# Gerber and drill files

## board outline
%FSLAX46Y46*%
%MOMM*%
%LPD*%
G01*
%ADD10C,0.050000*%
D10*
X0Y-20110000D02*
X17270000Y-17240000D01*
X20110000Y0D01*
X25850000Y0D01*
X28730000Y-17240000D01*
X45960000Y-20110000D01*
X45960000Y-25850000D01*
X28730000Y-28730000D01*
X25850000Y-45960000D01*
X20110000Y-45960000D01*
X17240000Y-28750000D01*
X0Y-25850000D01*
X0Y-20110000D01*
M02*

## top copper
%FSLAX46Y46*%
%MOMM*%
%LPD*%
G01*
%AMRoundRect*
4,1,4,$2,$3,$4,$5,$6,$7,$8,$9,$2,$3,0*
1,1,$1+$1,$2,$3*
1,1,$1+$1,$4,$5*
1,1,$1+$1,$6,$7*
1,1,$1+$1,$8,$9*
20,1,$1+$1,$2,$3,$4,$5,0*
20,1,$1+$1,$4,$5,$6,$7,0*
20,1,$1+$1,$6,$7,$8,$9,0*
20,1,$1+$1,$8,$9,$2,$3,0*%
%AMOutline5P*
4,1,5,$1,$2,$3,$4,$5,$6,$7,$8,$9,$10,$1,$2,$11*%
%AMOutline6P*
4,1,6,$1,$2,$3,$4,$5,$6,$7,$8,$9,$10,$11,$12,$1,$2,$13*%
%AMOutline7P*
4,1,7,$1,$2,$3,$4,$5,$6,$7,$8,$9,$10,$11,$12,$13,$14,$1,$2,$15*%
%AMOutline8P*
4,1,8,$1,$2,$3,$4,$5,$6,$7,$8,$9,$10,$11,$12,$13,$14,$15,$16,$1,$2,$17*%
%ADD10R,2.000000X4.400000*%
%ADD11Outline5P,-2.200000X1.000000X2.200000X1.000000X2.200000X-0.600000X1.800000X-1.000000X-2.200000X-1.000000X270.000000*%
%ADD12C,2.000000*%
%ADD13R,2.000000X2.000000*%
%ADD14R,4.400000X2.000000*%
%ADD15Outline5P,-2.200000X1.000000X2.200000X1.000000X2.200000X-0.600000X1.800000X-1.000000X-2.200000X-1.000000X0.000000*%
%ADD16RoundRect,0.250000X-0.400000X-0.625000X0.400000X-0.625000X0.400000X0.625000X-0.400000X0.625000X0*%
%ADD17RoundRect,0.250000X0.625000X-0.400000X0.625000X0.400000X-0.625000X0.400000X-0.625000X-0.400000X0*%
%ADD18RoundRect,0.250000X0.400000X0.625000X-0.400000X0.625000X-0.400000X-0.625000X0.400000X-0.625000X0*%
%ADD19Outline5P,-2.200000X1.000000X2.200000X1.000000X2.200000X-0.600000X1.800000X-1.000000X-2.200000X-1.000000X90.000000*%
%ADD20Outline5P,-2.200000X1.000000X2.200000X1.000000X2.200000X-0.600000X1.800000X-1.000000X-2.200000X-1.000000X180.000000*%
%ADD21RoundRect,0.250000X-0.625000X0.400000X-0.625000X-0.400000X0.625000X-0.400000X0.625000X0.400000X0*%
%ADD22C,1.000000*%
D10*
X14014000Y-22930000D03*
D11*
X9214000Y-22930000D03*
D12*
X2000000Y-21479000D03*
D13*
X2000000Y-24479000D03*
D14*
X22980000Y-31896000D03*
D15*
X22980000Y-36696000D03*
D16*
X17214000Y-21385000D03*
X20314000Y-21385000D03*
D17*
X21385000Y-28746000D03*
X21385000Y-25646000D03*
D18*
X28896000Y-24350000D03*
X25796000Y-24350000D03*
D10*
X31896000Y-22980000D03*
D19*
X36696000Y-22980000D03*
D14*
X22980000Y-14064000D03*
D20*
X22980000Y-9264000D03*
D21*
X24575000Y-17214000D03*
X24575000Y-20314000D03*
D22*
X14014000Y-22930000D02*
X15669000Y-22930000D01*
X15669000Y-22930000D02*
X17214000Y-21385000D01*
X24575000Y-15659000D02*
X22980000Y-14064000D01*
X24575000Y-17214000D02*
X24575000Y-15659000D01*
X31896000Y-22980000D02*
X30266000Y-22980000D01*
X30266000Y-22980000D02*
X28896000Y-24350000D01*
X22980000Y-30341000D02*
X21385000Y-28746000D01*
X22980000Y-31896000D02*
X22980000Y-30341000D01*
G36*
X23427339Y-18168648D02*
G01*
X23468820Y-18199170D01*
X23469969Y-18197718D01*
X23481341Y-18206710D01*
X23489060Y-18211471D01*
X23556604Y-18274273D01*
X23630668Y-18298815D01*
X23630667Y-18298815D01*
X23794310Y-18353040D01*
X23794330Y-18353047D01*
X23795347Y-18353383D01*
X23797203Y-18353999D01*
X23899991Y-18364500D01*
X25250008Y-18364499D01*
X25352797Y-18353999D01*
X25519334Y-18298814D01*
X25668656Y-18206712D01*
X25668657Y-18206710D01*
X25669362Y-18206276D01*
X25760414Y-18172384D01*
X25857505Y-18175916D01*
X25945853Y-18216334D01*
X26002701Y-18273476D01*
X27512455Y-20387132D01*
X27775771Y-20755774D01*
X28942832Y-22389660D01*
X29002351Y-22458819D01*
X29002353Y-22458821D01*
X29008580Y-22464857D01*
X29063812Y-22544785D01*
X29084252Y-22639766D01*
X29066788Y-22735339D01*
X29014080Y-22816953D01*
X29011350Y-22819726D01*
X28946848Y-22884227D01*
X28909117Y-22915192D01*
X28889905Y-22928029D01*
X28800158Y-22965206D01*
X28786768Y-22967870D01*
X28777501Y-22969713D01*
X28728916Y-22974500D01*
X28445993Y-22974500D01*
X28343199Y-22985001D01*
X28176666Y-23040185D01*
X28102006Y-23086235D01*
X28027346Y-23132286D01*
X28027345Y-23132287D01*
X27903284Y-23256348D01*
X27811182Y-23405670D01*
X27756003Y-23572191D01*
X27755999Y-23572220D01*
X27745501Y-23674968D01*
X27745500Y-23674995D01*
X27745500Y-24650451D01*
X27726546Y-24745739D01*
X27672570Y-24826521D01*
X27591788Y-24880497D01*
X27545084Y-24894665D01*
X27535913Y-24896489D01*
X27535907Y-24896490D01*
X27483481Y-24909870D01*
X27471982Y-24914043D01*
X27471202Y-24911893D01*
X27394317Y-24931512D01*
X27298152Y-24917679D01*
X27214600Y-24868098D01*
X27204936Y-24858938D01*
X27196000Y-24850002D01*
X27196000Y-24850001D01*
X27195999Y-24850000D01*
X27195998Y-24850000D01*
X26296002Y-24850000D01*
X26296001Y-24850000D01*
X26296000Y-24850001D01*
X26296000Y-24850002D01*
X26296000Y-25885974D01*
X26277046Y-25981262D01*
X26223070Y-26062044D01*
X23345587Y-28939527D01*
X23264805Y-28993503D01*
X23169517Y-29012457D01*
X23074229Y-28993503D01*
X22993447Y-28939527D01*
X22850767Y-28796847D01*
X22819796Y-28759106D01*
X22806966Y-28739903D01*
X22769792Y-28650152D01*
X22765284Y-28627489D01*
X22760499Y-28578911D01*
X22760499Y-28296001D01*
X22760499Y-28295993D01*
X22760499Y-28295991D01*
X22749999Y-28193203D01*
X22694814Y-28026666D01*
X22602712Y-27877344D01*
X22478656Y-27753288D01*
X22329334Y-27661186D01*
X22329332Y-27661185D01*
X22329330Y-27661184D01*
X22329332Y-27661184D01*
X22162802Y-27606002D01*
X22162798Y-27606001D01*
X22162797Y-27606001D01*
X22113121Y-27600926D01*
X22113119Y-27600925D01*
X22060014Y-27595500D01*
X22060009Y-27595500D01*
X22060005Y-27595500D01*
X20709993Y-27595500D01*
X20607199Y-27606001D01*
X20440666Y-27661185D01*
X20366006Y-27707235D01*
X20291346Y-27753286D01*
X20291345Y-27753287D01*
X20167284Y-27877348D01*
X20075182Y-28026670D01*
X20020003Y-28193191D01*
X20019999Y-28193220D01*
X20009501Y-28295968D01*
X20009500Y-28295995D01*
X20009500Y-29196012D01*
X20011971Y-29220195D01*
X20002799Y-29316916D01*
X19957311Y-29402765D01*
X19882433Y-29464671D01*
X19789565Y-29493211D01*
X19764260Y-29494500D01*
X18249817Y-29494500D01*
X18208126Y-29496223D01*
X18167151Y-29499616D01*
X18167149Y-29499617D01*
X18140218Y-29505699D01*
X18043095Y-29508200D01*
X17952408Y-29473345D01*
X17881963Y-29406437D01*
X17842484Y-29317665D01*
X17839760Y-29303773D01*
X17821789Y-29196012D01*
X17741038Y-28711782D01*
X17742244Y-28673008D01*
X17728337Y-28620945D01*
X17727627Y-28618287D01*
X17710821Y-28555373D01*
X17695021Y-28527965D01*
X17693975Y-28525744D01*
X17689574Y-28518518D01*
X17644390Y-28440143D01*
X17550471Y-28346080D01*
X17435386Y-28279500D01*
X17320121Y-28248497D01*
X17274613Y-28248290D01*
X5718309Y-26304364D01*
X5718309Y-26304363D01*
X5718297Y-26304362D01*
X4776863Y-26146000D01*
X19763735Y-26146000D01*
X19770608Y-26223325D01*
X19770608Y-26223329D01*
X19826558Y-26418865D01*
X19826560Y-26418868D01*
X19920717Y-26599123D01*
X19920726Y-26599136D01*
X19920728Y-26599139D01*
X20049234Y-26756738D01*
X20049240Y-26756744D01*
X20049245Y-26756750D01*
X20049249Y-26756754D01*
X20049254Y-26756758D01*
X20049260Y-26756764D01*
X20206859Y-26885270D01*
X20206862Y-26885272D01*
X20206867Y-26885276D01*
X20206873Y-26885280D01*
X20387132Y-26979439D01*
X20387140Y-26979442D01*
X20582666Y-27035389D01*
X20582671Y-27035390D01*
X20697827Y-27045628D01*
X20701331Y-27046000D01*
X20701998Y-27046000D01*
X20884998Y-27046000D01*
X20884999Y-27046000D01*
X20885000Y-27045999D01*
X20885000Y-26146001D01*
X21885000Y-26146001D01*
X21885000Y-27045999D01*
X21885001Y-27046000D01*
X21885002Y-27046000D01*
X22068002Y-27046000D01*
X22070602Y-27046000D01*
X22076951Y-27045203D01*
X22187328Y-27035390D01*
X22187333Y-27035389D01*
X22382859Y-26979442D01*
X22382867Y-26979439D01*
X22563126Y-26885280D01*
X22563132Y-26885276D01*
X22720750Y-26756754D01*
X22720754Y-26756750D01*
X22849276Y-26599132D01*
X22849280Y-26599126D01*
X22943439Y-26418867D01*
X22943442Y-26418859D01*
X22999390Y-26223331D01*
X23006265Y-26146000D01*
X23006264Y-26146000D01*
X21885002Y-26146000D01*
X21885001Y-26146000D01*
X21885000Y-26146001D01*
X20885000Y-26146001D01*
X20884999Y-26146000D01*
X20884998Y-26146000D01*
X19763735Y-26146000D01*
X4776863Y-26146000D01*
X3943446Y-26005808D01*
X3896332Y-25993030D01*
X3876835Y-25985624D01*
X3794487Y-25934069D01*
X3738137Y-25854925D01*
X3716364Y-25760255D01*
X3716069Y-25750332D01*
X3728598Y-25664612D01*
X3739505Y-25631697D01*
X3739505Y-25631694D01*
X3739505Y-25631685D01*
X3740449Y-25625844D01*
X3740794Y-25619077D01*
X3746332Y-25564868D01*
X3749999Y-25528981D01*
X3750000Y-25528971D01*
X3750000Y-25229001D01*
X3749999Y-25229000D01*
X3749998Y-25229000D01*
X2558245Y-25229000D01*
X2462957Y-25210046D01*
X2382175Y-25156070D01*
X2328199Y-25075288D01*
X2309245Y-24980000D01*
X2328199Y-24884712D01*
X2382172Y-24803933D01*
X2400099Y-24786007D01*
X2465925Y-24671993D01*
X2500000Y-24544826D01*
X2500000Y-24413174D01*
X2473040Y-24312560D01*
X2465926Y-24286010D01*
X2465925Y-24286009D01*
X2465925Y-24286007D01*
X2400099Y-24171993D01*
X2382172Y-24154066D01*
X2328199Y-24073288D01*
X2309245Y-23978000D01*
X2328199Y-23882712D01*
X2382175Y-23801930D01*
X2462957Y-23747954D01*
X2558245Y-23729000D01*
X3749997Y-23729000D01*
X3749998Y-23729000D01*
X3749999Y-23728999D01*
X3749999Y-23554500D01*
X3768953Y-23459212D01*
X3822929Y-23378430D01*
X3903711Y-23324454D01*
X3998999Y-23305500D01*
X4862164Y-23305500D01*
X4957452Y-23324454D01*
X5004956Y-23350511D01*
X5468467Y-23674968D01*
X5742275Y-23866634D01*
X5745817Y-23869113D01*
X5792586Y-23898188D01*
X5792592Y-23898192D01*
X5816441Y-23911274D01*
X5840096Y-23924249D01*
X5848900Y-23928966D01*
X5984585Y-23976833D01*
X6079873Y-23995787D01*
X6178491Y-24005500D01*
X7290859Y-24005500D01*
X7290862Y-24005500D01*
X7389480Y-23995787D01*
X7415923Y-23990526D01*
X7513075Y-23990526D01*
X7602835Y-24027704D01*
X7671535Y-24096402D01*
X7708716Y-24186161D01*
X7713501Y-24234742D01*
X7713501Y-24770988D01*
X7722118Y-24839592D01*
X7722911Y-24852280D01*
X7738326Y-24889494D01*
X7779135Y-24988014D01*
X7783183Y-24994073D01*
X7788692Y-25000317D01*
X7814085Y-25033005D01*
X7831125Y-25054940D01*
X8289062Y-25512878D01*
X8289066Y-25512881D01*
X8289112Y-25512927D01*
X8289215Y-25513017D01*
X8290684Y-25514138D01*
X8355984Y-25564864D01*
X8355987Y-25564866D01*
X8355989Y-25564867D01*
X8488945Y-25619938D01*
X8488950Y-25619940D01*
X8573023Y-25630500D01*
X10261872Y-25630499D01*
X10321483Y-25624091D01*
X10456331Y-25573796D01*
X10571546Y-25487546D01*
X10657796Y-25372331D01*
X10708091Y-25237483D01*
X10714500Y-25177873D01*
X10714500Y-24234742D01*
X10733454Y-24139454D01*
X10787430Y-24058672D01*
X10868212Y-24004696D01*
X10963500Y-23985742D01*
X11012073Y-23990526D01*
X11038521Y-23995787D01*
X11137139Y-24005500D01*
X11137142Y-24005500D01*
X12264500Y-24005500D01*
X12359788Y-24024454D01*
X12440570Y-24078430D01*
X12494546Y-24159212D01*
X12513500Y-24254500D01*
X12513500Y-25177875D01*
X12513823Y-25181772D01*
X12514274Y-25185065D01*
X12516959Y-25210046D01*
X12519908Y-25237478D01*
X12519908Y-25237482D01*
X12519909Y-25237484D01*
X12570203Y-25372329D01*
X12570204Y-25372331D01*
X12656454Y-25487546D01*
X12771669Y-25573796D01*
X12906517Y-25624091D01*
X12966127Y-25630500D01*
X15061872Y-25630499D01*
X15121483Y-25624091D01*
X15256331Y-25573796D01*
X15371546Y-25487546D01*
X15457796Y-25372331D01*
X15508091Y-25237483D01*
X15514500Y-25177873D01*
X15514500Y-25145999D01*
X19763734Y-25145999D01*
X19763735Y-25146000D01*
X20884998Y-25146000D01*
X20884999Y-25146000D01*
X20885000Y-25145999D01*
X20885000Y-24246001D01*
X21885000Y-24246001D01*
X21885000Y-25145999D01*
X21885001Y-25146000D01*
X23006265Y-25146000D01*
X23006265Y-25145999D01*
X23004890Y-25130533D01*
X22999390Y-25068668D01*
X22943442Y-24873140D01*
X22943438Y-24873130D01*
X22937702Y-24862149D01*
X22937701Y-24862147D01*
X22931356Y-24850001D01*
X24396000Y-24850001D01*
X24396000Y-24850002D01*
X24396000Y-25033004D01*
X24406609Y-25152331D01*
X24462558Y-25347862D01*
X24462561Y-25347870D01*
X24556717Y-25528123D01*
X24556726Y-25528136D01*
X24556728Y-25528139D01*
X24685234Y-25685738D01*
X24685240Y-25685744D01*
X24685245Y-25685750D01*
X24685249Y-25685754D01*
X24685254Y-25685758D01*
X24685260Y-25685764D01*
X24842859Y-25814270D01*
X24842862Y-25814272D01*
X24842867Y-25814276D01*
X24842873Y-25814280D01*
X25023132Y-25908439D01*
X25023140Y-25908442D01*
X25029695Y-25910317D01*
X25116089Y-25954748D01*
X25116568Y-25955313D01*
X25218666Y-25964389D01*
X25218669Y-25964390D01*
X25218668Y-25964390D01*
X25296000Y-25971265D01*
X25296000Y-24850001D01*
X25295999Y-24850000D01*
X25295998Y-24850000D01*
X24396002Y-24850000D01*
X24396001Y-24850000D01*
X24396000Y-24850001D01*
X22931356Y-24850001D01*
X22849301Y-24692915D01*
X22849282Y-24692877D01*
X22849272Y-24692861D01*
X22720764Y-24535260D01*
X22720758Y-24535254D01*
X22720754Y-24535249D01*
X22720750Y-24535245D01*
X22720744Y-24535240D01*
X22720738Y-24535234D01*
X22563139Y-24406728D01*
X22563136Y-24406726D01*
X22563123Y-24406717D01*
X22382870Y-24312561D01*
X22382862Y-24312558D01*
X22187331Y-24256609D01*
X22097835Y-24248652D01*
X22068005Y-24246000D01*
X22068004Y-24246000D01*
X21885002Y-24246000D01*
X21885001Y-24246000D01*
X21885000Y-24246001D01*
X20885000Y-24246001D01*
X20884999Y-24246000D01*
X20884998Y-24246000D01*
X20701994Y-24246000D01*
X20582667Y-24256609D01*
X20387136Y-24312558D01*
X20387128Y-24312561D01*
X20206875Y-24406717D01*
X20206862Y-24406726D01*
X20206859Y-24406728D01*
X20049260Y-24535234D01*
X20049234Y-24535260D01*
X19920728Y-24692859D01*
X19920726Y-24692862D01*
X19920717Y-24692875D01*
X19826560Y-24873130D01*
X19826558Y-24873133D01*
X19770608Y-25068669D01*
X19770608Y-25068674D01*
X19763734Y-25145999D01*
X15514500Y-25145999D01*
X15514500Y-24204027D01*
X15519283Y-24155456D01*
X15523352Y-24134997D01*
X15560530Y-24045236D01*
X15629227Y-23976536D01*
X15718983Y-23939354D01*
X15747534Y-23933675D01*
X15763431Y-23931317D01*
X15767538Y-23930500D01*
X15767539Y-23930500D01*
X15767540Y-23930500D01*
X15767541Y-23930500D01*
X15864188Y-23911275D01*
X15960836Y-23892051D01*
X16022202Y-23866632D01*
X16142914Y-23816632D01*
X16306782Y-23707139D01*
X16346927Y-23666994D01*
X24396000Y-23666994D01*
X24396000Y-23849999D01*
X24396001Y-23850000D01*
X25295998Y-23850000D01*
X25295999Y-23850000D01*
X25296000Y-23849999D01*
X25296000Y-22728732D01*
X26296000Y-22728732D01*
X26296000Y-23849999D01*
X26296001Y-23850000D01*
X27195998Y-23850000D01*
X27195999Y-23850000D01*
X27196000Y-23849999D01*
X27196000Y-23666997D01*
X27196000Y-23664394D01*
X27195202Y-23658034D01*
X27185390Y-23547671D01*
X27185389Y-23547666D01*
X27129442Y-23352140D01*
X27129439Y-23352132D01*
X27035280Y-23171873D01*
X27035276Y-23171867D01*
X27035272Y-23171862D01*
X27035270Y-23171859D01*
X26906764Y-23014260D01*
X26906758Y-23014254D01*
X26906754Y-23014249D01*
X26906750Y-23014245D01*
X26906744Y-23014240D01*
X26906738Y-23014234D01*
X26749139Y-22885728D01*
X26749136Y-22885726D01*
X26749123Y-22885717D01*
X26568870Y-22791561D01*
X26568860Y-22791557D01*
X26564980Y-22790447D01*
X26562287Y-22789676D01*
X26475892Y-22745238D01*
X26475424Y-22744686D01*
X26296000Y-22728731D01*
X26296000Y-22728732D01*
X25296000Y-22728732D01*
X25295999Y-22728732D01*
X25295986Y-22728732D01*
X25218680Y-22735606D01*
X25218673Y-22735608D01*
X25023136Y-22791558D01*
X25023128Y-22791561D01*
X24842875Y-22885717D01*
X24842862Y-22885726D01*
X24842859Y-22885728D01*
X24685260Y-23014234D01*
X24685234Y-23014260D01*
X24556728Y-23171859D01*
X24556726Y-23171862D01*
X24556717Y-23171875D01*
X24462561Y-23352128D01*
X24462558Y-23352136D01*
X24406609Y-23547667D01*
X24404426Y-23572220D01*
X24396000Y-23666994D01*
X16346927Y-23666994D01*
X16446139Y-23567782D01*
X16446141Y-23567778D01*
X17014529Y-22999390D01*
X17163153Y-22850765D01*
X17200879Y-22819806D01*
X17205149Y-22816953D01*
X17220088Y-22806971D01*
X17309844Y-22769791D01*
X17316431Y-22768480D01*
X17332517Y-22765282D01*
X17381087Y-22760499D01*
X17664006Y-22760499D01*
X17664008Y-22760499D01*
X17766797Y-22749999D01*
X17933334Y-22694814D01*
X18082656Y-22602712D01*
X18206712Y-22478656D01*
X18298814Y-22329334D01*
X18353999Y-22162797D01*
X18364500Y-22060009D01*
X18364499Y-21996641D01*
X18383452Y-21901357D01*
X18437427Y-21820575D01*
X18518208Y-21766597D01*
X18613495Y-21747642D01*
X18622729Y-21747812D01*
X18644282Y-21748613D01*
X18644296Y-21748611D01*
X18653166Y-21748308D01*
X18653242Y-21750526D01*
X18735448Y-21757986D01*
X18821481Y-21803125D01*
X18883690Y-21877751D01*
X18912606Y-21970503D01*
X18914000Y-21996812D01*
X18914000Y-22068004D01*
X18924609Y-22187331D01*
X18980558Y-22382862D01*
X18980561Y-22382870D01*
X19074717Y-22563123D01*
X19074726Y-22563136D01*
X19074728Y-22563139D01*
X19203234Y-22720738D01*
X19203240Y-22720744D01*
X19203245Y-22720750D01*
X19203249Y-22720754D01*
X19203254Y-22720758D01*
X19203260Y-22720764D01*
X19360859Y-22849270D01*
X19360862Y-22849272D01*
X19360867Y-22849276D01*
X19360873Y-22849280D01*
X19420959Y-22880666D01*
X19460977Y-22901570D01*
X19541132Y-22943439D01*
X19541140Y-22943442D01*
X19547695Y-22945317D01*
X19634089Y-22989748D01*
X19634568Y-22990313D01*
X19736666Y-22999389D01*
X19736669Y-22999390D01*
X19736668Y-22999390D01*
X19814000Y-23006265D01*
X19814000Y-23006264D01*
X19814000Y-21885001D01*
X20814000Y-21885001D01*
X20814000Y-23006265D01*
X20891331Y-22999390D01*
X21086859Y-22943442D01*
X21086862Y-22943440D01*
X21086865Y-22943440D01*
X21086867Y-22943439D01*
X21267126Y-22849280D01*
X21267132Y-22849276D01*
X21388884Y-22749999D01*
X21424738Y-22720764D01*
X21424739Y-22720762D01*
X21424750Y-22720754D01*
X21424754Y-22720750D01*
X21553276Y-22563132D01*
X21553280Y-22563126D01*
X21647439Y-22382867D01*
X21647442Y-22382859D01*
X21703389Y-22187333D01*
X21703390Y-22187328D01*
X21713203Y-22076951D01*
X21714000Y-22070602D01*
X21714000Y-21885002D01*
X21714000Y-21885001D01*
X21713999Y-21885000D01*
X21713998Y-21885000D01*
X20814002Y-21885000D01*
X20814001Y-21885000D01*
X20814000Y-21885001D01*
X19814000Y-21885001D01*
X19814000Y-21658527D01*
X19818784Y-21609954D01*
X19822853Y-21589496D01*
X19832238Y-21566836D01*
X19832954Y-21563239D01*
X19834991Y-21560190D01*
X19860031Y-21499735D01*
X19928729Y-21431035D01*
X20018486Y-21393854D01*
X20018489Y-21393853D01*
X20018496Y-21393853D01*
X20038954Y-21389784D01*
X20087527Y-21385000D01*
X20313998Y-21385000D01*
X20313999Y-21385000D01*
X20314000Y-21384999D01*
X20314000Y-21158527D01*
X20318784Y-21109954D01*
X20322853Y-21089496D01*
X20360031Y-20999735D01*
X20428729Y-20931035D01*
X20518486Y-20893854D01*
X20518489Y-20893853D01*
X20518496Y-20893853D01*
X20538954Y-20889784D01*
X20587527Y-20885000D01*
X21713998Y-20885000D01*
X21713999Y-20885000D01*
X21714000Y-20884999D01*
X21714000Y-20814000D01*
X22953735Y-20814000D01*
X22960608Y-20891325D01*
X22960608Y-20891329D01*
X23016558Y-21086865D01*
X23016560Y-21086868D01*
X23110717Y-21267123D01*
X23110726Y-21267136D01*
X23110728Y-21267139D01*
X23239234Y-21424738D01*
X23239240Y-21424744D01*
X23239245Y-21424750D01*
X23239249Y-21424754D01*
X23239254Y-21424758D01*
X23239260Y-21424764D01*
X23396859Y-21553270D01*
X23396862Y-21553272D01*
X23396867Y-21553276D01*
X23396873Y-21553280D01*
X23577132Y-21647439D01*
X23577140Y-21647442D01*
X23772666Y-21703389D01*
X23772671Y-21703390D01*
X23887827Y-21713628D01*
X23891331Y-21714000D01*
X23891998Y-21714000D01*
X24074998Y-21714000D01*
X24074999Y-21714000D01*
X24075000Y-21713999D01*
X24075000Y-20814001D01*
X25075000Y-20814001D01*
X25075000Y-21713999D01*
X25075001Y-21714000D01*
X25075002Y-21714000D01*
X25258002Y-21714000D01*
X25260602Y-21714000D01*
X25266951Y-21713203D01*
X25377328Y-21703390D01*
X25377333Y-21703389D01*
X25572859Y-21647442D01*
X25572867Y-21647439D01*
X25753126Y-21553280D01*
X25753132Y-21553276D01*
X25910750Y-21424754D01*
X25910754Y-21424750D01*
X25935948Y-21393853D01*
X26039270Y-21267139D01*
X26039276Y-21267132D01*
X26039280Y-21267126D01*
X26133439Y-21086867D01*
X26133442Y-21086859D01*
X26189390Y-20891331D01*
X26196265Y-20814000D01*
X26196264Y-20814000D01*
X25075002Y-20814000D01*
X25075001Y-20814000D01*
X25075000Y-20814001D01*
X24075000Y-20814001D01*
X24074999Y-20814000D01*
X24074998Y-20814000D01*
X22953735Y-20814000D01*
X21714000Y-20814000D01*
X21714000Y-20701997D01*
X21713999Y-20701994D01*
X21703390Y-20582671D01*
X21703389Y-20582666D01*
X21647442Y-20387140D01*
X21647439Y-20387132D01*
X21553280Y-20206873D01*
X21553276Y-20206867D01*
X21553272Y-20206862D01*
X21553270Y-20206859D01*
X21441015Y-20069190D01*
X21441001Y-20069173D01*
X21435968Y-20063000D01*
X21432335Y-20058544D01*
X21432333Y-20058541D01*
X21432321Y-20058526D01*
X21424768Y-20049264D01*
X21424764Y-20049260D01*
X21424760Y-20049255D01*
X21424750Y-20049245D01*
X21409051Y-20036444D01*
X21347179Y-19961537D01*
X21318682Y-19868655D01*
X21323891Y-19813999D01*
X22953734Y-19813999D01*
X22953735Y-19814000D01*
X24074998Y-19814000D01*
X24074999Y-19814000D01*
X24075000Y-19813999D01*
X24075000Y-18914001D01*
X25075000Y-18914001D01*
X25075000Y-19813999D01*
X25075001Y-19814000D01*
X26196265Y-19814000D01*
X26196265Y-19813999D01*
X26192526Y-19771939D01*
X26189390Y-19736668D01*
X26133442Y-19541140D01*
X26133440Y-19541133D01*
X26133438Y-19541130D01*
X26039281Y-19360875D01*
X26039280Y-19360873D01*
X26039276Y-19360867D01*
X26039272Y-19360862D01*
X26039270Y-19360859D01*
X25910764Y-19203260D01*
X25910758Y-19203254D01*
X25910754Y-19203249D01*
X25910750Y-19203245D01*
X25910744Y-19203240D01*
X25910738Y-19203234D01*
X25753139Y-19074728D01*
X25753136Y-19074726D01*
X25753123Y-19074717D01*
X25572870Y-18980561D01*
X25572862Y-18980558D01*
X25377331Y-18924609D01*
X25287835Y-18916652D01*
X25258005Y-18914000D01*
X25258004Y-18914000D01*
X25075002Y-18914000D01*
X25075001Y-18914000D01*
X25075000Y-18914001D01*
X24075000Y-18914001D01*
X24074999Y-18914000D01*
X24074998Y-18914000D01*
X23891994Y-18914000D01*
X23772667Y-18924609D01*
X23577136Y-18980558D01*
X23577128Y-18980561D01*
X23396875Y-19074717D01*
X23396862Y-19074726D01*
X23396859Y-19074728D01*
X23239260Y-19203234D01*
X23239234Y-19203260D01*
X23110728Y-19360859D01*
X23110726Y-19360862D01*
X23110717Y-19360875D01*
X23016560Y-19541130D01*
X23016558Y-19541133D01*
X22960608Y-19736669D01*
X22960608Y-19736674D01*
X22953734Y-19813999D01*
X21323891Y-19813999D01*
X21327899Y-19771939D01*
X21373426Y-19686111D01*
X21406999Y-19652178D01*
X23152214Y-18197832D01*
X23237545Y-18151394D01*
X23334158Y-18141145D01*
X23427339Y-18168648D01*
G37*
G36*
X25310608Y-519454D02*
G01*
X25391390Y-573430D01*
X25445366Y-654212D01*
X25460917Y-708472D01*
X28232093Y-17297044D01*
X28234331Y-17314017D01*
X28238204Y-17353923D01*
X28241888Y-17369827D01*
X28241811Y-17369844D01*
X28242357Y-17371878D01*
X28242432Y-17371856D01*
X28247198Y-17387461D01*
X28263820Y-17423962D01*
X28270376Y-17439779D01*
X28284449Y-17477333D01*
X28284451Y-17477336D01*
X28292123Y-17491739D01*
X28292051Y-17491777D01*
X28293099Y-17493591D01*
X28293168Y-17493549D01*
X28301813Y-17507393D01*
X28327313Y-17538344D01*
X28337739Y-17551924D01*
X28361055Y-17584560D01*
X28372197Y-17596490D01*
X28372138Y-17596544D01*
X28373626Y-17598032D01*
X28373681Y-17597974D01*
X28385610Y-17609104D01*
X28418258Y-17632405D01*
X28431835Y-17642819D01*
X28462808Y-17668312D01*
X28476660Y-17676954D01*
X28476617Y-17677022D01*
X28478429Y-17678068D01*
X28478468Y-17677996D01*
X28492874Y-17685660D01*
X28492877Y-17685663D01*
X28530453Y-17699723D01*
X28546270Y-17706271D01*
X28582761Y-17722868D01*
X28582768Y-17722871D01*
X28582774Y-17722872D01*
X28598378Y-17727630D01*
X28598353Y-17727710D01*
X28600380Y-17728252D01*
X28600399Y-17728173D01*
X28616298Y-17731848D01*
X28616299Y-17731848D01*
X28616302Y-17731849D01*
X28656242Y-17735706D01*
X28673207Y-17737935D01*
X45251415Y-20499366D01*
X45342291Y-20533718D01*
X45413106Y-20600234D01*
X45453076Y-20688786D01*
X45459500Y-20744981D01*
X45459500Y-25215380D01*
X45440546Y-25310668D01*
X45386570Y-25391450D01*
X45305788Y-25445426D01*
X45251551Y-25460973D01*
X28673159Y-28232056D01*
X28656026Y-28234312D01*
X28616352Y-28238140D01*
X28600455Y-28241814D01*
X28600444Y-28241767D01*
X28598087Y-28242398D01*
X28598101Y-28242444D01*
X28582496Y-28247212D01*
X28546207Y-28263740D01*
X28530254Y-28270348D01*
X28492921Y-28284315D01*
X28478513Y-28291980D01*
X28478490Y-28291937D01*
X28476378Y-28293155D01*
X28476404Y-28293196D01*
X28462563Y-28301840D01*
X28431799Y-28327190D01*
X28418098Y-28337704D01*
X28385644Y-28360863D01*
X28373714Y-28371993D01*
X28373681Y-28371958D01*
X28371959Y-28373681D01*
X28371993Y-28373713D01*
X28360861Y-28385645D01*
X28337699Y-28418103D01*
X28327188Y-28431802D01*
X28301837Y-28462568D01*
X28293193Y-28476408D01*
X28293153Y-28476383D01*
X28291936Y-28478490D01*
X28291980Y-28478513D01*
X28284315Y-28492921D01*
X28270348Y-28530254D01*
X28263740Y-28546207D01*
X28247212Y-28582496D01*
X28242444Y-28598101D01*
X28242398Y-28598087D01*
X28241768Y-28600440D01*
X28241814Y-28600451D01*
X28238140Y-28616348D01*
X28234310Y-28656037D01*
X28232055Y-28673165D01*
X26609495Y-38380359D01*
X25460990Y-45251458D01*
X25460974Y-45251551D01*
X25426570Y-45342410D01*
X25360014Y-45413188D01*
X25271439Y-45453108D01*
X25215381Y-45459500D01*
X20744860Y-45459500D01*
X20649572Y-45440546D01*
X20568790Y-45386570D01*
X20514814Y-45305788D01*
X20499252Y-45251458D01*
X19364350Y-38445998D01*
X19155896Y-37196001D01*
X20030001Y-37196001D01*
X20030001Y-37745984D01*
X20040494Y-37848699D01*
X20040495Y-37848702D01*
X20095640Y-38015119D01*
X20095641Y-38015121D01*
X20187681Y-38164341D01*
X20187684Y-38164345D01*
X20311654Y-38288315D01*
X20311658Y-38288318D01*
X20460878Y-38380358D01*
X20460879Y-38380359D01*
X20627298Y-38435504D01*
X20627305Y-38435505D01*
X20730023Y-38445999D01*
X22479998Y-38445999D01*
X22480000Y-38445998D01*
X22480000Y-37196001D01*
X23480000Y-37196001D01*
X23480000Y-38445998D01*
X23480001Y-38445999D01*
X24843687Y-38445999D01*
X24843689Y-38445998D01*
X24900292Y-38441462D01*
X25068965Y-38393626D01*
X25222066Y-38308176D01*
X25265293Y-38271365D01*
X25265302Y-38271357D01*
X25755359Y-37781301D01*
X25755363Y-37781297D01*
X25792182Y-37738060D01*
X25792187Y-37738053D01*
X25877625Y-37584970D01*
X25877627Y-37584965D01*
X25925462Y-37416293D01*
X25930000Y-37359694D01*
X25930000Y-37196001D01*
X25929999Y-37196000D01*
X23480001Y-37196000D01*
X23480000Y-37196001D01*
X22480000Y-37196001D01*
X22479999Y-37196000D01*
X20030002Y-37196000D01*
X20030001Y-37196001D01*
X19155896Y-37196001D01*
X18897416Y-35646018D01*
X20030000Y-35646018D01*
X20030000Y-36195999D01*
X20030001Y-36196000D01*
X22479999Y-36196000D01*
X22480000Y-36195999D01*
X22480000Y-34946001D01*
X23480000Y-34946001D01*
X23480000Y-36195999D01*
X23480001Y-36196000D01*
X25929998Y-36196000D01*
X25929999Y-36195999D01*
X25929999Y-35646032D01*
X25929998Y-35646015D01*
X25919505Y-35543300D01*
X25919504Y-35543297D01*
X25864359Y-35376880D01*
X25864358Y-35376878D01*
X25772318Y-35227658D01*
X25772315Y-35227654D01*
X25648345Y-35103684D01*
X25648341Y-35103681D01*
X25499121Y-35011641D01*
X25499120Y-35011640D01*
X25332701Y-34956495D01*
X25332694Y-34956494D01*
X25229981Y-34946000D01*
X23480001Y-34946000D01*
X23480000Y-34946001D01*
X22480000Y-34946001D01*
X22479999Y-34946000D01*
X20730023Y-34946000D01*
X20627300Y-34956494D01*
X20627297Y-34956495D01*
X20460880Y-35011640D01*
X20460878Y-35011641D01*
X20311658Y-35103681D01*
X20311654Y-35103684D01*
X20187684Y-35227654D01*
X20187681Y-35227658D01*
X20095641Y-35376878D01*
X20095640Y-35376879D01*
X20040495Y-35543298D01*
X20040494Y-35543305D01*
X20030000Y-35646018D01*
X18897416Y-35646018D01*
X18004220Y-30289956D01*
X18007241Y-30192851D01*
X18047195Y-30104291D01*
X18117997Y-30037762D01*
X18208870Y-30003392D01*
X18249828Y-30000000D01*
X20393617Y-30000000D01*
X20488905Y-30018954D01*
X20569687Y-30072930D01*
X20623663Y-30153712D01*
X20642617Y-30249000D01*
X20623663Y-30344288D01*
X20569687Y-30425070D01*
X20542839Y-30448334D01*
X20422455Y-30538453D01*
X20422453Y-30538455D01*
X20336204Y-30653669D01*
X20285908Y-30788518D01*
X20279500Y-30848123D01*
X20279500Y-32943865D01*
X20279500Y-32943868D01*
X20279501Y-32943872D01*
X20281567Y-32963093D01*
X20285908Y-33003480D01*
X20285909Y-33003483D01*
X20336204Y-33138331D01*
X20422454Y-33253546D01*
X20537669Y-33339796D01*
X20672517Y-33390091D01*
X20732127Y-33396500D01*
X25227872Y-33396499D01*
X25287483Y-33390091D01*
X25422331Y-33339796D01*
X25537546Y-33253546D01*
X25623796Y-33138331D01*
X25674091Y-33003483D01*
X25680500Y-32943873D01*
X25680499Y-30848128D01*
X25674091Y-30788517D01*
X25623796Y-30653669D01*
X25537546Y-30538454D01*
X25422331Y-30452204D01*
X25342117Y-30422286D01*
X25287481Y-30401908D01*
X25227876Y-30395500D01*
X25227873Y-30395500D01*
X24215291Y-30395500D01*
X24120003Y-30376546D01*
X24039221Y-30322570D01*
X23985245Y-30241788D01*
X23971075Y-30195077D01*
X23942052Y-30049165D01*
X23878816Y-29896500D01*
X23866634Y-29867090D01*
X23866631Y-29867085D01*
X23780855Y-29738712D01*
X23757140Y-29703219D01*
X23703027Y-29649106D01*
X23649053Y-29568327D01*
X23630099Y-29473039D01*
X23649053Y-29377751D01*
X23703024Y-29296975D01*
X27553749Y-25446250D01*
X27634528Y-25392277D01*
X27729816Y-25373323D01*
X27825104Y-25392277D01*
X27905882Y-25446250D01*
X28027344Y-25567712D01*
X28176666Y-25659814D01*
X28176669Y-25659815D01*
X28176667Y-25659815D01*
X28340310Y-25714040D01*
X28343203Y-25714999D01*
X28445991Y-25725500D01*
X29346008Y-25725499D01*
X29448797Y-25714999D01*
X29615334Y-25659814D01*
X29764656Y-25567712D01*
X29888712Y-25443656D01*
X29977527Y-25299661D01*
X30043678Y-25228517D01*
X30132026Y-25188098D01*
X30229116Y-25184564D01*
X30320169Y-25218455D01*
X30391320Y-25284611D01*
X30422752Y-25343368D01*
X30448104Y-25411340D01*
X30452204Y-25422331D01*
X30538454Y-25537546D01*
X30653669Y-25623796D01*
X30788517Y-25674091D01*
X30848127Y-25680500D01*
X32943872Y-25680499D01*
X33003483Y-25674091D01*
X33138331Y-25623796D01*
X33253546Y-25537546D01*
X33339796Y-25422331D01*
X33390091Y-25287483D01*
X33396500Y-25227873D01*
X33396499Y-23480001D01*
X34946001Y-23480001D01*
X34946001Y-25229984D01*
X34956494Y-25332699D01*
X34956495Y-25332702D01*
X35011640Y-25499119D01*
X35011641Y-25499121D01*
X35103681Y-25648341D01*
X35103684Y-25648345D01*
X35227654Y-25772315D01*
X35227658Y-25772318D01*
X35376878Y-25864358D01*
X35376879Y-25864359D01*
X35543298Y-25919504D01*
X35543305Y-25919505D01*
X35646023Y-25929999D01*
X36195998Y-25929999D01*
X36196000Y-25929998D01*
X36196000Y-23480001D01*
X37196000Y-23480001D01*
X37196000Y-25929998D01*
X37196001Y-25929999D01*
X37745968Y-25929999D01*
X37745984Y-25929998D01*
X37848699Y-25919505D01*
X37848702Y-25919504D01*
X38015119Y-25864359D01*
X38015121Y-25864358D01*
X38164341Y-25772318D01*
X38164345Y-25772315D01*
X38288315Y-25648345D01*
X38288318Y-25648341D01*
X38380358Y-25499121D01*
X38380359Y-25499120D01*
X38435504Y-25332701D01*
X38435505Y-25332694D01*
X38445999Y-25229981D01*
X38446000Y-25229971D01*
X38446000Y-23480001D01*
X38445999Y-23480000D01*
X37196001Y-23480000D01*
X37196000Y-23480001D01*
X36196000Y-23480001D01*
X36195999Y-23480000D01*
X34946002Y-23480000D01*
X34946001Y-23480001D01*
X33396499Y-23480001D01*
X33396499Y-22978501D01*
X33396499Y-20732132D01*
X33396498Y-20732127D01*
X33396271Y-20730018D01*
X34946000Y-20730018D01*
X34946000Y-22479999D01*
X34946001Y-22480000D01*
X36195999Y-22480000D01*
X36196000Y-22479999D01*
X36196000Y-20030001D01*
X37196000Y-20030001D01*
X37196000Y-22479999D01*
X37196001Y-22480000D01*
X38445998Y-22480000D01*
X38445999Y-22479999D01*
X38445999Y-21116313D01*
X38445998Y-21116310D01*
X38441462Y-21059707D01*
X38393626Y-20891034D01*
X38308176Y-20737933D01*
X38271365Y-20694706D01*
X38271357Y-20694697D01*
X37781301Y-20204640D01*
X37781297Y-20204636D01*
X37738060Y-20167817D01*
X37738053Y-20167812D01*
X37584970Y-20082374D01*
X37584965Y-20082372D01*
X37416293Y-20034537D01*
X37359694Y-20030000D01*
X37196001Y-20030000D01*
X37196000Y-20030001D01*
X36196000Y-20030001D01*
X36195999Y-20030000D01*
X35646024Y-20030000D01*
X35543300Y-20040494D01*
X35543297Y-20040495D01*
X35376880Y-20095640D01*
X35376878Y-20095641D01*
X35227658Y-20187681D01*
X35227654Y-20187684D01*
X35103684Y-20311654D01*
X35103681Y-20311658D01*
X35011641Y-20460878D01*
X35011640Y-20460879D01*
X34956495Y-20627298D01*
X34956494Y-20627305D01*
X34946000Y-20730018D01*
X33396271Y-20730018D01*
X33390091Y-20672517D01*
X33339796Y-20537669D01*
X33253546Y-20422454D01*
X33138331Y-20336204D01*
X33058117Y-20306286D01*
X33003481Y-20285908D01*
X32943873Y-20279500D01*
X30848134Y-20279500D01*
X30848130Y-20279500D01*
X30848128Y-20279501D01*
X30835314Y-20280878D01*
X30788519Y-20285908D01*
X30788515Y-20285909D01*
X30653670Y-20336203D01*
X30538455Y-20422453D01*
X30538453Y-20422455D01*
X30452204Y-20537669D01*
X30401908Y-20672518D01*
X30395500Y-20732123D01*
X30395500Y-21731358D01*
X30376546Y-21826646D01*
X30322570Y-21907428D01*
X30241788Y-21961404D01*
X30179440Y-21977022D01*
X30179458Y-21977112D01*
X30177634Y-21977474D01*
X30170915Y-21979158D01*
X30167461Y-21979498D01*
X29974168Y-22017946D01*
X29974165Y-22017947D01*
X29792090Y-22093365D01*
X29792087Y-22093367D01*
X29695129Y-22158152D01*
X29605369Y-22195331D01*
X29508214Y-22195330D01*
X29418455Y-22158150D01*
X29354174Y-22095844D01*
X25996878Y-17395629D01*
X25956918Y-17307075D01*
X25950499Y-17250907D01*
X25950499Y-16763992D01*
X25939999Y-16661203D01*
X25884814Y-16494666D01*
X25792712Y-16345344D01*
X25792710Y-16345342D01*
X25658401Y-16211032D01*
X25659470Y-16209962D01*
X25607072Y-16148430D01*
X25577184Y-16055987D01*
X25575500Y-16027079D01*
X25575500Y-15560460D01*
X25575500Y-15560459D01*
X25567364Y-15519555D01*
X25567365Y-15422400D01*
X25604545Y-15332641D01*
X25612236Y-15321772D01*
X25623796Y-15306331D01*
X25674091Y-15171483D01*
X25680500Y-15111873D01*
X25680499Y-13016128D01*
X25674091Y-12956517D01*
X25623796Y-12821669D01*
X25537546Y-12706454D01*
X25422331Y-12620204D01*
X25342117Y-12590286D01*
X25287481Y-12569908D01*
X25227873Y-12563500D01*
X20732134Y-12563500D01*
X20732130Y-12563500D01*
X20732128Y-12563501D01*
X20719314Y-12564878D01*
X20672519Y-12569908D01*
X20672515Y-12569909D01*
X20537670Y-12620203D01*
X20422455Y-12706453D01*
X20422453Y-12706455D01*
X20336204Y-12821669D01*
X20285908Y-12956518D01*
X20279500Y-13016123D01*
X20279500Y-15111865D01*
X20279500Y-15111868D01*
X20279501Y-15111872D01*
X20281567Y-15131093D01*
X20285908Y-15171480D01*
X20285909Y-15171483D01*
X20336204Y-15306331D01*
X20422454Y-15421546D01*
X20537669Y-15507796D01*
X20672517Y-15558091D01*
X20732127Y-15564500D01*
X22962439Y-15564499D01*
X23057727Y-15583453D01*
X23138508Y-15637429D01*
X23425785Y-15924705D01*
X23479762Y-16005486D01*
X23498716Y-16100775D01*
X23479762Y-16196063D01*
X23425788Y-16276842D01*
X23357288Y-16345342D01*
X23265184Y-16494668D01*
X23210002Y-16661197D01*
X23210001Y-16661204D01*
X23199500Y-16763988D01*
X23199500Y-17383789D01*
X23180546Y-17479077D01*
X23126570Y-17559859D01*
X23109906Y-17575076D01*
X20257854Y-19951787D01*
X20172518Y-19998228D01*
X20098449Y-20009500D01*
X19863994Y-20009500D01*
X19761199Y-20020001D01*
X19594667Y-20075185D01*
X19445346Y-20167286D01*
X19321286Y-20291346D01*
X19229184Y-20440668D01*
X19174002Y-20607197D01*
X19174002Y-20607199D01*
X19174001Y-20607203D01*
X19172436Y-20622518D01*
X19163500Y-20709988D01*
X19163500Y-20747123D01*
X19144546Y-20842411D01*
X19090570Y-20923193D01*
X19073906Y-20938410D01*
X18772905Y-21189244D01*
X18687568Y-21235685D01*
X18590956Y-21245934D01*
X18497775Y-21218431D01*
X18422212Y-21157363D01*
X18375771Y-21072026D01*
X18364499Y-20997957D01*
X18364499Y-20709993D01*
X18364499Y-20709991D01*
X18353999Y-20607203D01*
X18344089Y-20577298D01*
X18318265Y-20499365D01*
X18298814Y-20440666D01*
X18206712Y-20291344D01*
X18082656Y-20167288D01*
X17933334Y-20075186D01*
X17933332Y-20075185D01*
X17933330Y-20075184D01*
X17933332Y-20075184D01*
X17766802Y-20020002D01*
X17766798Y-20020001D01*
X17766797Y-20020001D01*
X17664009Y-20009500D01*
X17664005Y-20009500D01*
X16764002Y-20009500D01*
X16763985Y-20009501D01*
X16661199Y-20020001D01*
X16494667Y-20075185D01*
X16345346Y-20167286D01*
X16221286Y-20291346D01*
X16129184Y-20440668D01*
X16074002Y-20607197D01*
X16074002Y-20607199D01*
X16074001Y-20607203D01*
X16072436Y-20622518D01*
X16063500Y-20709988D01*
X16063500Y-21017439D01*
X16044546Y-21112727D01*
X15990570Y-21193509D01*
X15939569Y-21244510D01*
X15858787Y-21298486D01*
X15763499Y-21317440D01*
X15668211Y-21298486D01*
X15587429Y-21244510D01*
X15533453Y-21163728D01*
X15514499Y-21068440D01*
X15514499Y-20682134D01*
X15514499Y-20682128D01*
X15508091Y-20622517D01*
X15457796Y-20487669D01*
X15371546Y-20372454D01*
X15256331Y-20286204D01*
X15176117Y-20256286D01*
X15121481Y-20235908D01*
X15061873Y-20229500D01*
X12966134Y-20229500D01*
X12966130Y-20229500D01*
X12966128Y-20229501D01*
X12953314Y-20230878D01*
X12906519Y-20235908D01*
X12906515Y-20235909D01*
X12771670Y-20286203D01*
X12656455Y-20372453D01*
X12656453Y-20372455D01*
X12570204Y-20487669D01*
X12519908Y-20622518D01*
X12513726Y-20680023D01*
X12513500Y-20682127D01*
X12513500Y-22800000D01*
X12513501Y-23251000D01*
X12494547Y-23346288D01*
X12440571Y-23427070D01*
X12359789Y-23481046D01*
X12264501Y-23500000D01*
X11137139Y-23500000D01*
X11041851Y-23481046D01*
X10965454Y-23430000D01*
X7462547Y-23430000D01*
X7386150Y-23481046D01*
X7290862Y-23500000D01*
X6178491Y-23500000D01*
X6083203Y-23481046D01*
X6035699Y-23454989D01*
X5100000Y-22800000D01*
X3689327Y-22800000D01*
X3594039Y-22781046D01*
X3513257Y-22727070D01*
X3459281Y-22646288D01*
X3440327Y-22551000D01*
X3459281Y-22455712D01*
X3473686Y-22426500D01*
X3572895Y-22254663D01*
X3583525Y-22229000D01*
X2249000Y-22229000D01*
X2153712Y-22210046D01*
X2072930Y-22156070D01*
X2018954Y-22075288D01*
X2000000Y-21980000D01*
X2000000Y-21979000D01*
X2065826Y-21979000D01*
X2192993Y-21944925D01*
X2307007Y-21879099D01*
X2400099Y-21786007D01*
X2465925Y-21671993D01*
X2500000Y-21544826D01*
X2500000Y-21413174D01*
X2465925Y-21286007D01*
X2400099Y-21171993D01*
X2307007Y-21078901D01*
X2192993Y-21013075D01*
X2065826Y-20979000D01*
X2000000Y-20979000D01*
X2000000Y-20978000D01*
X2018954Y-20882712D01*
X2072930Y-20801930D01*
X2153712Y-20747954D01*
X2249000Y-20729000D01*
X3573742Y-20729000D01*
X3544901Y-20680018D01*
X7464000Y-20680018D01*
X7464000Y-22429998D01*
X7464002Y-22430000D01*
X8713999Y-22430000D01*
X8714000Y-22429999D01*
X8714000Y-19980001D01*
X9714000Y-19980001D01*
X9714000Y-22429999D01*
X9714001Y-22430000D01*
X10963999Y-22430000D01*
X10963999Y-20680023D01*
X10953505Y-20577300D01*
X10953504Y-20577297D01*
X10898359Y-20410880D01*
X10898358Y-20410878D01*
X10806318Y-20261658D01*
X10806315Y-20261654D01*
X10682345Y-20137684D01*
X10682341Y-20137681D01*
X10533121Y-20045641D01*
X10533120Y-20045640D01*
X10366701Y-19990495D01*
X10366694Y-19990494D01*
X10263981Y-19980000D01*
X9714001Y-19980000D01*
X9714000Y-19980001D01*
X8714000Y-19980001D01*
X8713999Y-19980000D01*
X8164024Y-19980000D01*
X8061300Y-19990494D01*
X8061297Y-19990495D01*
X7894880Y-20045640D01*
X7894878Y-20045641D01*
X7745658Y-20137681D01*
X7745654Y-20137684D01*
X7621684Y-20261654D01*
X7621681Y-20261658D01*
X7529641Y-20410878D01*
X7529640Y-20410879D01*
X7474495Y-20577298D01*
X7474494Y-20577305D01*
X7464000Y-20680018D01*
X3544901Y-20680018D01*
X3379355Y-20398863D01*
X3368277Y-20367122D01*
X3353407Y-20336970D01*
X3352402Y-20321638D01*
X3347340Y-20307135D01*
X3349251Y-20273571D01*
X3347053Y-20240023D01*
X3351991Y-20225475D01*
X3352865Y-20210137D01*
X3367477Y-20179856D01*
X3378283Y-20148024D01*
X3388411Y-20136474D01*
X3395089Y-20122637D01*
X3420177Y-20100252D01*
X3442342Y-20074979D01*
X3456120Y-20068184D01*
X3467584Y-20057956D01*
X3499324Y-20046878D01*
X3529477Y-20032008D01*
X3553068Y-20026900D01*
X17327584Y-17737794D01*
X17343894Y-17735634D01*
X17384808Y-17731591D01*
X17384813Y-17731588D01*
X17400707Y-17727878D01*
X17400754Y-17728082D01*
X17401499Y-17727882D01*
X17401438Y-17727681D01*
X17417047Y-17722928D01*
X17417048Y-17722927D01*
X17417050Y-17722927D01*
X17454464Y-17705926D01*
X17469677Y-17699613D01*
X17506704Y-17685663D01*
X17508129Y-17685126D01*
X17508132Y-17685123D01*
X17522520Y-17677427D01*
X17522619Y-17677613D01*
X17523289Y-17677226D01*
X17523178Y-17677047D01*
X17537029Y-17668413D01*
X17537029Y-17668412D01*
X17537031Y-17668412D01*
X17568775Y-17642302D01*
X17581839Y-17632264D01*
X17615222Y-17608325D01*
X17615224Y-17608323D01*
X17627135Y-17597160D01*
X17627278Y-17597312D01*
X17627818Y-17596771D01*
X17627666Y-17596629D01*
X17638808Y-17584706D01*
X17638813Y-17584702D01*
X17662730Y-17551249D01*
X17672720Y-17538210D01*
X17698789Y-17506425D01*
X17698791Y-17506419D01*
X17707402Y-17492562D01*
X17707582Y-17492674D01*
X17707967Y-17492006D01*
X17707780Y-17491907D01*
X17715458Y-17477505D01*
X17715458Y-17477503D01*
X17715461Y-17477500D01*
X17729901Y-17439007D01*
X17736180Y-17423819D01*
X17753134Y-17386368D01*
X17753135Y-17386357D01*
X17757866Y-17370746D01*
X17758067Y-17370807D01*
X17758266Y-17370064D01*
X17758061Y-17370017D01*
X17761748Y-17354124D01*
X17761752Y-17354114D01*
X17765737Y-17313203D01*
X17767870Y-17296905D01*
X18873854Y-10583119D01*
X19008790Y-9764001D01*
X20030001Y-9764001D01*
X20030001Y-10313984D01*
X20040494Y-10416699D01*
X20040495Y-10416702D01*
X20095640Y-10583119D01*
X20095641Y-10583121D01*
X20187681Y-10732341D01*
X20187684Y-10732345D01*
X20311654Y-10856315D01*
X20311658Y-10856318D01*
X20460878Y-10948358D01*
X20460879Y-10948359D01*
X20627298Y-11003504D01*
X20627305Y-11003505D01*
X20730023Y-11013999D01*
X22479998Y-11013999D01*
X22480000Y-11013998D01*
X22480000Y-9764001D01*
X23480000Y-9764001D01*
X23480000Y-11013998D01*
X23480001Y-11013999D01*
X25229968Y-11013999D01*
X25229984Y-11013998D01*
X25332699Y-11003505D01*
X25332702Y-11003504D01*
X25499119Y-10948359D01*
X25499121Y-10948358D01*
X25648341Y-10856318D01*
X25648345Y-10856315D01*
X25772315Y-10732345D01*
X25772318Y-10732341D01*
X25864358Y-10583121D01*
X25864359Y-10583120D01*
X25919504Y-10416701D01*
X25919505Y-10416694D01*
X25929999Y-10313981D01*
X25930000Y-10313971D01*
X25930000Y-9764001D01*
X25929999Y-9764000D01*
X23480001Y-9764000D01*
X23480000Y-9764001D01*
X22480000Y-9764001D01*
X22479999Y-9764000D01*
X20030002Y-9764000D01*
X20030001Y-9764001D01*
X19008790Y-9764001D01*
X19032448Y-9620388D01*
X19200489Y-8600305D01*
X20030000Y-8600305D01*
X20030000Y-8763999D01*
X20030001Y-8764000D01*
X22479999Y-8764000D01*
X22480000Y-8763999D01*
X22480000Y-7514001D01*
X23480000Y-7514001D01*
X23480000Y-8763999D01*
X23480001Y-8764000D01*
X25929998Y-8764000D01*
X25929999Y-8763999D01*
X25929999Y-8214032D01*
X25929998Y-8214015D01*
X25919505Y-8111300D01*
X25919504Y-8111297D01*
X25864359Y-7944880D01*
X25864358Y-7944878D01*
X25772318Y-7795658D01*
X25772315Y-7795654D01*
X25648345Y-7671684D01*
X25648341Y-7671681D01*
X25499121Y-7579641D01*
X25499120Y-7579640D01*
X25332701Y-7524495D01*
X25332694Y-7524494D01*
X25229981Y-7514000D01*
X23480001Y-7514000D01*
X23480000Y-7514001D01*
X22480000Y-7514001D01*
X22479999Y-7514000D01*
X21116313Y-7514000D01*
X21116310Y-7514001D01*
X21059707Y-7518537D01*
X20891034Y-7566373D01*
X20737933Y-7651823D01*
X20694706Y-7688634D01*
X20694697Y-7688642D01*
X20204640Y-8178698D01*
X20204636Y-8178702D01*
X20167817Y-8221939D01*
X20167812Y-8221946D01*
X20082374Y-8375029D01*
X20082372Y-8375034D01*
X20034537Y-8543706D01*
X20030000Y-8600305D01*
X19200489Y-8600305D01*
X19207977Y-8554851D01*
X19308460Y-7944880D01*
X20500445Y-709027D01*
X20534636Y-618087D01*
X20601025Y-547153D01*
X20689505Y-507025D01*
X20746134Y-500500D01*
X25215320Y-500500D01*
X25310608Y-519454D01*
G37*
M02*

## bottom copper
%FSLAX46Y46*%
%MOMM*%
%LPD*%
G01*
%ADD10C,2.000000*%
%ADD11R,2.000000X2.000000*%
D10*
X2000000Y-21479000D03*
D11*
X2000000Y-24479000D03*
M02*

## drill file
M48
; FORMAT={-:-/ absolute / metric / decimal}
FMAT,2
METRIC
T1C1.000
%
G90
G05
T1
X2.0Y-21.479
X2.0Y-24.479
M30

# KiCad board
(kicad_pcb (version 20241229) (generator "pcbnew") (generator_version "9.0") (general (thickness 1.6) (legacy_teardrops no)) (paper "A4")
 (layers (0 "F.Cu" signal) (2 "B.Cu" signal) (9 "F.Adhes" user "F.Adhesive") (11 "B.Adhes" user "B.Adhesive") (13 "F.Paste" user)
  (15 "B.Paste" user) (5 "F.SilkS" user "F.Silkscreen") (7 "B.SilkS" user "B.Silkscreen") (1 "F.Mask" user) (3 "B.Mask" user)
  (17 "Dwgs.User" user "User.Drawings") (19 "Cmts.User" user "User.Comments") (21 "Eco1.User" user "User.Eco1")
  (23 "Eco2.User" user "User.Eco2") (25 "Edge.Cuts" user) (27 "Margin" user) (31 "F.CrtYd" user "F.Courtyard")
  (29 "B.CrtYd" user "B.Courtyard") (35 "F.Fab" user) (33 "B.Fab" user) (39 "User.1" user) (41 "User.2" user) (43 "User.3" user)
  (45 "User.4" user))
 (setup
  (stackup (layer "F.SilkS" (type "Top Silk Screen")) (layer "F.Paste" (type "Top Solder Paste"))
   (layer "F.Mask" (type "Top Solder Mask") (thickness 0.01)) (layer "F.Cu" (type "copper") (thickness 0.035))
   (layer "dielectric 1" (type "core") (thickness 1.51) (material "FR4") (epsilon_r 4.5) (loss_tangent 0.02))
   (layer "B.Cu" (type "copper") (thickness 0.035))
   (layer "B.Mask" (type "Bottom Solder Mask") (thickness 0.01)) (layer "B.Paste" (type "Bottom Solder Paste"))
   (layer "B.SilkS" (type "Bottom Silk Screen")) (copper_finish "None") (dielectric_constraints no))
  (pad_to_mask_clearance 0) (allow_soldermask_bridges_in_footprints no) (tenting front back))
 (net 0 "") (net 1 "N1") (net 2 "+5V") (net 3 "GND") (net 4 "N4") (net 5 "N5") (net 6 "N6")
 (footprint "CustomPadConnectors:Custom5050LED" (layer "F.Cu") (at 11.614 22.93 180)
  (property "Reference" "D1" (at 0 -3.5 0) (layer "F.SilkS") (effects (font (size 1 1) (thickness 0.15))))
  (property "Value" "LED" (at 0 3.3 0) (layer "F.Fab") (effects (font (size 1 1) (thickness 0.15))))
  (pad "1" smd rect (at -2.4 0 270) (size 4.4 2) (layers "F.Cu" "F.Mask" "F.Paste") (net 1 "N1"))
  (pad "2" smd roundrect (at 2.4 0 270) (size 4.4 2) (layers "F.Cu" "F.Mask" "F.Paste") (roundrect_rratio 0) (chamfer_ratio 0.2)
   (chamfer bottom_right) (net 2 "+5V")))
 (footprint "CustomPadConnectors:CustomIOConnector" (layer "F.Cu") (at 2 22.979 -90)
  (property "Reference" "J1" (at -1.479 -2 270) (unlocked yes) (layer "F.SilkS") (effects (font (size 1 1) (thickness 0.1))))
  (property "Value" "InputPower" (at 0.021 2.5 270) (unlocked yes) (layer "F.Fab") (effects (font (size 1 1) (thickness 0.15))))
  (pad "1" thru_hole circle (at -1.5 0 270) (size 2 2) (drill 1) (layers "*.Cu" "*.Mask") (remove_unused_layers no) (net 2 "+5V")
   (thermal_bridge_width 1.5) (thermal_bridge_angle 0))
  (pad "2" thru_hole rect (at 1.5 0 270) (size 2 2) (drill 1) (layers "*.Cu" "*.Mask") (remove_unused_layers no) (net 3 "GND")
   (thermal_bridge_width 1.5)))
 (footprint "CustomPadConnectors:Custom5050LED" (layer "F.Cu") (at 22.98 34.296 -90)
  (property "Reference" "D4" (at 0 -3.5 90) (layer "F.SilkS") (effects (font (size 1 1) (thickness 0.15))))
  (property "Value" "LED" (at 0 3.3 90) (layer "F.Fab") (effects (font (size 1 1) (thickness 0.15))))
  (pad "1" smd rect (at -2.4 0) (size 4.4 2) (layers "F.Cu" "F.Mask" "F.Paste") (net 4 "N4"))
  (pad "2" smd roundrect (at 2.4 0) (size 4.4 2) (layers "F.Cu" "F.Mask" "F.Paste") (roundrect_rratio 0) (chamfer_ratio 0.2)
   (chamfer bottom_right) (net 2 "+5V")))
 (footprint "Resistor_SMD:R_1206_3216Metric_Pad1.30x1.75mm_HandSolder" (layer "F.Cu") (at 18.764 21.385)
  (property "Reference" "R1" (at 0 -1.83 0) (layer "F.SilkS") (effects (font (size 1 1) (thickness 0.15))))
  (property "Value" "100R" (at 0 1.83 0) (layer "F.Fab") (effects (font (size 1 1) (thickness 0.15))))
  (pad "1" smd roundrect (at -1.55 0) (size 1.3 1.75) (layers "F.Cu" "F.Mask" "F.Paste") (roundrect_rratio 0.192308) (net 1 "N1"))
  (pad "2" smd roundrect (at 1.55 0) (size 1.3 1.75) (layers "F.Cu" "F.Mask" "F.Paste") (roundrect_rratio 0.192308) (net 3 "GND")))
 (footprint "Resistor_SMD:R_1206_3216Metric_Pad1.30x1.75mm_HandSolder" (layer "F.Cu") (at 21.385 27.196 90)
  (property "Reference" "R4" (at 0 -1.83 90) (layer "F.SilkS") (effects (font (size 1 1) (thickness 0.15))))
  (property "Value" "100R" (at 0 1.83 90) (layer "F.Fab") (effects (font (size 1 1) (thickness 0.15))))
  (pad "1" smd roundrect (at -1.55 0 90) (size 1.3 1.75) (layers "F.Cu" "F.Mask" "F.Paste") (roundrect_rratio 0.192308) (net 4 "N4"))
  (pad "2" smd roundrect (at 1.55 0 90) (size 1.3 1.75) (layers "F.Cu" "F.Mask" "F.Paste") (roundrect_rratio 0.192308) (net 3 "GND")))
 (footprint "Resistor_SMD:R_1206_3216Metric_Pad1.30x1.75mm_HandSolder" (layer "F.Cu") (at 27.346 24.35 180)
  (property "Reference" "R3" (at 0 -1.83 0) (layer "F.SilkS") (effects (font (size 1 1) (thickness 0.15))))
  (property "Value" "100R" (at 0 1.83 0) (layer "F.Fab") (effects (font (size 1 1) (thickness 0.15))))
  (pad "1" smd roundrect (at -1.55 0 180) (size 1.3 1.75) (layers "F.Cu" "F.Mask" "F.Paste") (roundrect_rratio 0.192308) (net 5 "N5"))
  (pad "2" smd roundrect (at 1.55 0 180) (size 1.3 1.75) (layers "F.Cu" "F.Mask" "F.Paste") (roundrect_rratio 0.192308) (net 3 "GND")))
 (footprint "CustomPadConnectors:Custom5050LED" (layer "F.Cu") (at 34.296 22.98)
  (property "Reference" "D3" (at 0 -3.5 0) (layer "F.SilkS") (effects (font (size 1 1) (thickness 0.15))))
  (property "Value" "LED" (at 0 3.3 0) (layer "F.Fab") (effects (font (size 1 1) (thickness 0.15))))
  (pad "1" smd rect (at -2.4 0 90) (size 4.4 2) (layers "F.Cu" "F.Mask" "F.Paste") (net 5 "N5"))
  (pad "2" smd roundrect (at 2.4 0 90) (size 4.4 2) (layers "F.Cu" "F.Mask" "F.Paste") (roundrect_rratio 0) (chamfer_ratio 0.2)
   (chamfer bottom_right) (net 2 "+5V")))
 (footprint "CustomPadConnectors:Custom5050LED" (layer "F.Cu") (at 22.98 11.664 90)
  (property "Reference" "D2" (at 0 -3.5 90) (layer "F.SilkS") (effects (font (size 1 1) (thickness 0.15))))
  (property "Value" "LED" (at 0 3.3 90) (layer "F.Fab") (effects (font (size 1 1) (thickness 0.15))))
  (pad "1" smd rect (at -2.4 0 180) (size 4.4 2) (layers "F.Cu" "F.Mask" "F.Paste") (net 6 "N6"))
  (pad "2" smd roundrect (at 2.4 0 180) (size 4.4 2) (layers "F.Cu" "F.Mask" "F.Paste") (roundrect_rratio 0) (chamfer_ratio 0.2)
   (chamfer bottom_right) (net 2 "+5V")))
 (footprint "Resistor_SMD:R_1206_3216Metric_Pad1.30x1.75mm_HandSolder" (layer "F.Cu") (at 24.575 18.764 -90)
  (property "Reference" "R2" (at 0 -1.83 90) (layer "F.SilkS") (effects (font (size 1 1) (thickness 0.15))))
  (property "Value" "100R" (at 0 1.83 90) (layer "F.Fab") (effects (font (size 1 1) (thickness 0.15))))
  (pad "1" smd roundrect (at -1.55 0 270) (size 1.3 1.75) (layers "F.Cu" "F.Mask" "F.Paste") (roundrect_rratio 0.192308) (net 6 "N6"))
  (pad "2" smd roundrect (at 1.55 0 270) (size 1.3 1.75) (layers "F.Cu" "F.Mask" "F.Paste") (roundrect_rratio 0.192308) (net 3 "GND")))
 (gr_poly
  (pts (xy 0 20.11) (xy 17.27 17.24) (xy 20.11 0) (xy 25.85 0) (xy 28.73 17.24) (xy 45.96 20.11) (xy 45.96 25.85) (xy 28.73 28.73)
   (xy 25.85 45.96) (xy 20.11 45.96) (xy 17.24 28.75) (xy 0 25.85))
  (stroke (width 0.05) (type solid)) (fill no) (layer "Edge.Cuts"))
 (segment (start 14.014 22.93) (end 15.669 22.93) (width 1) (layer "F.Cu") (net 1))
 (segment (start 15.669 22.93) (end 17.214 21.385) (width 1) (layer "F.Cu") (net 1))
 (segment (start 24.575 15.659) (end 22.98 14.064) (width 1) (layer "F.Cu") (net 6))
 (segment (start 24.575 17.214) (end 24.575 15.659) (width 1) (layer "F.Cu") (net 6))
 (segment (start 31.896 22.98) (end 30.266 22.98) (width 1) (layer "F.Cu") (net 5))
 (segment (start 30.266 22.98) (end 28.896 24.35) (width 1) (layer "F.Cu") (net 5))
 (segment (start 22.98 30.341) (end 21.385 28.746) (width 1) (layer "F.Cu") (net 4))
 (segment (start 22.98 31.896) (end 22.98 30.341) (width 1) (layer "F.Cu") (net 4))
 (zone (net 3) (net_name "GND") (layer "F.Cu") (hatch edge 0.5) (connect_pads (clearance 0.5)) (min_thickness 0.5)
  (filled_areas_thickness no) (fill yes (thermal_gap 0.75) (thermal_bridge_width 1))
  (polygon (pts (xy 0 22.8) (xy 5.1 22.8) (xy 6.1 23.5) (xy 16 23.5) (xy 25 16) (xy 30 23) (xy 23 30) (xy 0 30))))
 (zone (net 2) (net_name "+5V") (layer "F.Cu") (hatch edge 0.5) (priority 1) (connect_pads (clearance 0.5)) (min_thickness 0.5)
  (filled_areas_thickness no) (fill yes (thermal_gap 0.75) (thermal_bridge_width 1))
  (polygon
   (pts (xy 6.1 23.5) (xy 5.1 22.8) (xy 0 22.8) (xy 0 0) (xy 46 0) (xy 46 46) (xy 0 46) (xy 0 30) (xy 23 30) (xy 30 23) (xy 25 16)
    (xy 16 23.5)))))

